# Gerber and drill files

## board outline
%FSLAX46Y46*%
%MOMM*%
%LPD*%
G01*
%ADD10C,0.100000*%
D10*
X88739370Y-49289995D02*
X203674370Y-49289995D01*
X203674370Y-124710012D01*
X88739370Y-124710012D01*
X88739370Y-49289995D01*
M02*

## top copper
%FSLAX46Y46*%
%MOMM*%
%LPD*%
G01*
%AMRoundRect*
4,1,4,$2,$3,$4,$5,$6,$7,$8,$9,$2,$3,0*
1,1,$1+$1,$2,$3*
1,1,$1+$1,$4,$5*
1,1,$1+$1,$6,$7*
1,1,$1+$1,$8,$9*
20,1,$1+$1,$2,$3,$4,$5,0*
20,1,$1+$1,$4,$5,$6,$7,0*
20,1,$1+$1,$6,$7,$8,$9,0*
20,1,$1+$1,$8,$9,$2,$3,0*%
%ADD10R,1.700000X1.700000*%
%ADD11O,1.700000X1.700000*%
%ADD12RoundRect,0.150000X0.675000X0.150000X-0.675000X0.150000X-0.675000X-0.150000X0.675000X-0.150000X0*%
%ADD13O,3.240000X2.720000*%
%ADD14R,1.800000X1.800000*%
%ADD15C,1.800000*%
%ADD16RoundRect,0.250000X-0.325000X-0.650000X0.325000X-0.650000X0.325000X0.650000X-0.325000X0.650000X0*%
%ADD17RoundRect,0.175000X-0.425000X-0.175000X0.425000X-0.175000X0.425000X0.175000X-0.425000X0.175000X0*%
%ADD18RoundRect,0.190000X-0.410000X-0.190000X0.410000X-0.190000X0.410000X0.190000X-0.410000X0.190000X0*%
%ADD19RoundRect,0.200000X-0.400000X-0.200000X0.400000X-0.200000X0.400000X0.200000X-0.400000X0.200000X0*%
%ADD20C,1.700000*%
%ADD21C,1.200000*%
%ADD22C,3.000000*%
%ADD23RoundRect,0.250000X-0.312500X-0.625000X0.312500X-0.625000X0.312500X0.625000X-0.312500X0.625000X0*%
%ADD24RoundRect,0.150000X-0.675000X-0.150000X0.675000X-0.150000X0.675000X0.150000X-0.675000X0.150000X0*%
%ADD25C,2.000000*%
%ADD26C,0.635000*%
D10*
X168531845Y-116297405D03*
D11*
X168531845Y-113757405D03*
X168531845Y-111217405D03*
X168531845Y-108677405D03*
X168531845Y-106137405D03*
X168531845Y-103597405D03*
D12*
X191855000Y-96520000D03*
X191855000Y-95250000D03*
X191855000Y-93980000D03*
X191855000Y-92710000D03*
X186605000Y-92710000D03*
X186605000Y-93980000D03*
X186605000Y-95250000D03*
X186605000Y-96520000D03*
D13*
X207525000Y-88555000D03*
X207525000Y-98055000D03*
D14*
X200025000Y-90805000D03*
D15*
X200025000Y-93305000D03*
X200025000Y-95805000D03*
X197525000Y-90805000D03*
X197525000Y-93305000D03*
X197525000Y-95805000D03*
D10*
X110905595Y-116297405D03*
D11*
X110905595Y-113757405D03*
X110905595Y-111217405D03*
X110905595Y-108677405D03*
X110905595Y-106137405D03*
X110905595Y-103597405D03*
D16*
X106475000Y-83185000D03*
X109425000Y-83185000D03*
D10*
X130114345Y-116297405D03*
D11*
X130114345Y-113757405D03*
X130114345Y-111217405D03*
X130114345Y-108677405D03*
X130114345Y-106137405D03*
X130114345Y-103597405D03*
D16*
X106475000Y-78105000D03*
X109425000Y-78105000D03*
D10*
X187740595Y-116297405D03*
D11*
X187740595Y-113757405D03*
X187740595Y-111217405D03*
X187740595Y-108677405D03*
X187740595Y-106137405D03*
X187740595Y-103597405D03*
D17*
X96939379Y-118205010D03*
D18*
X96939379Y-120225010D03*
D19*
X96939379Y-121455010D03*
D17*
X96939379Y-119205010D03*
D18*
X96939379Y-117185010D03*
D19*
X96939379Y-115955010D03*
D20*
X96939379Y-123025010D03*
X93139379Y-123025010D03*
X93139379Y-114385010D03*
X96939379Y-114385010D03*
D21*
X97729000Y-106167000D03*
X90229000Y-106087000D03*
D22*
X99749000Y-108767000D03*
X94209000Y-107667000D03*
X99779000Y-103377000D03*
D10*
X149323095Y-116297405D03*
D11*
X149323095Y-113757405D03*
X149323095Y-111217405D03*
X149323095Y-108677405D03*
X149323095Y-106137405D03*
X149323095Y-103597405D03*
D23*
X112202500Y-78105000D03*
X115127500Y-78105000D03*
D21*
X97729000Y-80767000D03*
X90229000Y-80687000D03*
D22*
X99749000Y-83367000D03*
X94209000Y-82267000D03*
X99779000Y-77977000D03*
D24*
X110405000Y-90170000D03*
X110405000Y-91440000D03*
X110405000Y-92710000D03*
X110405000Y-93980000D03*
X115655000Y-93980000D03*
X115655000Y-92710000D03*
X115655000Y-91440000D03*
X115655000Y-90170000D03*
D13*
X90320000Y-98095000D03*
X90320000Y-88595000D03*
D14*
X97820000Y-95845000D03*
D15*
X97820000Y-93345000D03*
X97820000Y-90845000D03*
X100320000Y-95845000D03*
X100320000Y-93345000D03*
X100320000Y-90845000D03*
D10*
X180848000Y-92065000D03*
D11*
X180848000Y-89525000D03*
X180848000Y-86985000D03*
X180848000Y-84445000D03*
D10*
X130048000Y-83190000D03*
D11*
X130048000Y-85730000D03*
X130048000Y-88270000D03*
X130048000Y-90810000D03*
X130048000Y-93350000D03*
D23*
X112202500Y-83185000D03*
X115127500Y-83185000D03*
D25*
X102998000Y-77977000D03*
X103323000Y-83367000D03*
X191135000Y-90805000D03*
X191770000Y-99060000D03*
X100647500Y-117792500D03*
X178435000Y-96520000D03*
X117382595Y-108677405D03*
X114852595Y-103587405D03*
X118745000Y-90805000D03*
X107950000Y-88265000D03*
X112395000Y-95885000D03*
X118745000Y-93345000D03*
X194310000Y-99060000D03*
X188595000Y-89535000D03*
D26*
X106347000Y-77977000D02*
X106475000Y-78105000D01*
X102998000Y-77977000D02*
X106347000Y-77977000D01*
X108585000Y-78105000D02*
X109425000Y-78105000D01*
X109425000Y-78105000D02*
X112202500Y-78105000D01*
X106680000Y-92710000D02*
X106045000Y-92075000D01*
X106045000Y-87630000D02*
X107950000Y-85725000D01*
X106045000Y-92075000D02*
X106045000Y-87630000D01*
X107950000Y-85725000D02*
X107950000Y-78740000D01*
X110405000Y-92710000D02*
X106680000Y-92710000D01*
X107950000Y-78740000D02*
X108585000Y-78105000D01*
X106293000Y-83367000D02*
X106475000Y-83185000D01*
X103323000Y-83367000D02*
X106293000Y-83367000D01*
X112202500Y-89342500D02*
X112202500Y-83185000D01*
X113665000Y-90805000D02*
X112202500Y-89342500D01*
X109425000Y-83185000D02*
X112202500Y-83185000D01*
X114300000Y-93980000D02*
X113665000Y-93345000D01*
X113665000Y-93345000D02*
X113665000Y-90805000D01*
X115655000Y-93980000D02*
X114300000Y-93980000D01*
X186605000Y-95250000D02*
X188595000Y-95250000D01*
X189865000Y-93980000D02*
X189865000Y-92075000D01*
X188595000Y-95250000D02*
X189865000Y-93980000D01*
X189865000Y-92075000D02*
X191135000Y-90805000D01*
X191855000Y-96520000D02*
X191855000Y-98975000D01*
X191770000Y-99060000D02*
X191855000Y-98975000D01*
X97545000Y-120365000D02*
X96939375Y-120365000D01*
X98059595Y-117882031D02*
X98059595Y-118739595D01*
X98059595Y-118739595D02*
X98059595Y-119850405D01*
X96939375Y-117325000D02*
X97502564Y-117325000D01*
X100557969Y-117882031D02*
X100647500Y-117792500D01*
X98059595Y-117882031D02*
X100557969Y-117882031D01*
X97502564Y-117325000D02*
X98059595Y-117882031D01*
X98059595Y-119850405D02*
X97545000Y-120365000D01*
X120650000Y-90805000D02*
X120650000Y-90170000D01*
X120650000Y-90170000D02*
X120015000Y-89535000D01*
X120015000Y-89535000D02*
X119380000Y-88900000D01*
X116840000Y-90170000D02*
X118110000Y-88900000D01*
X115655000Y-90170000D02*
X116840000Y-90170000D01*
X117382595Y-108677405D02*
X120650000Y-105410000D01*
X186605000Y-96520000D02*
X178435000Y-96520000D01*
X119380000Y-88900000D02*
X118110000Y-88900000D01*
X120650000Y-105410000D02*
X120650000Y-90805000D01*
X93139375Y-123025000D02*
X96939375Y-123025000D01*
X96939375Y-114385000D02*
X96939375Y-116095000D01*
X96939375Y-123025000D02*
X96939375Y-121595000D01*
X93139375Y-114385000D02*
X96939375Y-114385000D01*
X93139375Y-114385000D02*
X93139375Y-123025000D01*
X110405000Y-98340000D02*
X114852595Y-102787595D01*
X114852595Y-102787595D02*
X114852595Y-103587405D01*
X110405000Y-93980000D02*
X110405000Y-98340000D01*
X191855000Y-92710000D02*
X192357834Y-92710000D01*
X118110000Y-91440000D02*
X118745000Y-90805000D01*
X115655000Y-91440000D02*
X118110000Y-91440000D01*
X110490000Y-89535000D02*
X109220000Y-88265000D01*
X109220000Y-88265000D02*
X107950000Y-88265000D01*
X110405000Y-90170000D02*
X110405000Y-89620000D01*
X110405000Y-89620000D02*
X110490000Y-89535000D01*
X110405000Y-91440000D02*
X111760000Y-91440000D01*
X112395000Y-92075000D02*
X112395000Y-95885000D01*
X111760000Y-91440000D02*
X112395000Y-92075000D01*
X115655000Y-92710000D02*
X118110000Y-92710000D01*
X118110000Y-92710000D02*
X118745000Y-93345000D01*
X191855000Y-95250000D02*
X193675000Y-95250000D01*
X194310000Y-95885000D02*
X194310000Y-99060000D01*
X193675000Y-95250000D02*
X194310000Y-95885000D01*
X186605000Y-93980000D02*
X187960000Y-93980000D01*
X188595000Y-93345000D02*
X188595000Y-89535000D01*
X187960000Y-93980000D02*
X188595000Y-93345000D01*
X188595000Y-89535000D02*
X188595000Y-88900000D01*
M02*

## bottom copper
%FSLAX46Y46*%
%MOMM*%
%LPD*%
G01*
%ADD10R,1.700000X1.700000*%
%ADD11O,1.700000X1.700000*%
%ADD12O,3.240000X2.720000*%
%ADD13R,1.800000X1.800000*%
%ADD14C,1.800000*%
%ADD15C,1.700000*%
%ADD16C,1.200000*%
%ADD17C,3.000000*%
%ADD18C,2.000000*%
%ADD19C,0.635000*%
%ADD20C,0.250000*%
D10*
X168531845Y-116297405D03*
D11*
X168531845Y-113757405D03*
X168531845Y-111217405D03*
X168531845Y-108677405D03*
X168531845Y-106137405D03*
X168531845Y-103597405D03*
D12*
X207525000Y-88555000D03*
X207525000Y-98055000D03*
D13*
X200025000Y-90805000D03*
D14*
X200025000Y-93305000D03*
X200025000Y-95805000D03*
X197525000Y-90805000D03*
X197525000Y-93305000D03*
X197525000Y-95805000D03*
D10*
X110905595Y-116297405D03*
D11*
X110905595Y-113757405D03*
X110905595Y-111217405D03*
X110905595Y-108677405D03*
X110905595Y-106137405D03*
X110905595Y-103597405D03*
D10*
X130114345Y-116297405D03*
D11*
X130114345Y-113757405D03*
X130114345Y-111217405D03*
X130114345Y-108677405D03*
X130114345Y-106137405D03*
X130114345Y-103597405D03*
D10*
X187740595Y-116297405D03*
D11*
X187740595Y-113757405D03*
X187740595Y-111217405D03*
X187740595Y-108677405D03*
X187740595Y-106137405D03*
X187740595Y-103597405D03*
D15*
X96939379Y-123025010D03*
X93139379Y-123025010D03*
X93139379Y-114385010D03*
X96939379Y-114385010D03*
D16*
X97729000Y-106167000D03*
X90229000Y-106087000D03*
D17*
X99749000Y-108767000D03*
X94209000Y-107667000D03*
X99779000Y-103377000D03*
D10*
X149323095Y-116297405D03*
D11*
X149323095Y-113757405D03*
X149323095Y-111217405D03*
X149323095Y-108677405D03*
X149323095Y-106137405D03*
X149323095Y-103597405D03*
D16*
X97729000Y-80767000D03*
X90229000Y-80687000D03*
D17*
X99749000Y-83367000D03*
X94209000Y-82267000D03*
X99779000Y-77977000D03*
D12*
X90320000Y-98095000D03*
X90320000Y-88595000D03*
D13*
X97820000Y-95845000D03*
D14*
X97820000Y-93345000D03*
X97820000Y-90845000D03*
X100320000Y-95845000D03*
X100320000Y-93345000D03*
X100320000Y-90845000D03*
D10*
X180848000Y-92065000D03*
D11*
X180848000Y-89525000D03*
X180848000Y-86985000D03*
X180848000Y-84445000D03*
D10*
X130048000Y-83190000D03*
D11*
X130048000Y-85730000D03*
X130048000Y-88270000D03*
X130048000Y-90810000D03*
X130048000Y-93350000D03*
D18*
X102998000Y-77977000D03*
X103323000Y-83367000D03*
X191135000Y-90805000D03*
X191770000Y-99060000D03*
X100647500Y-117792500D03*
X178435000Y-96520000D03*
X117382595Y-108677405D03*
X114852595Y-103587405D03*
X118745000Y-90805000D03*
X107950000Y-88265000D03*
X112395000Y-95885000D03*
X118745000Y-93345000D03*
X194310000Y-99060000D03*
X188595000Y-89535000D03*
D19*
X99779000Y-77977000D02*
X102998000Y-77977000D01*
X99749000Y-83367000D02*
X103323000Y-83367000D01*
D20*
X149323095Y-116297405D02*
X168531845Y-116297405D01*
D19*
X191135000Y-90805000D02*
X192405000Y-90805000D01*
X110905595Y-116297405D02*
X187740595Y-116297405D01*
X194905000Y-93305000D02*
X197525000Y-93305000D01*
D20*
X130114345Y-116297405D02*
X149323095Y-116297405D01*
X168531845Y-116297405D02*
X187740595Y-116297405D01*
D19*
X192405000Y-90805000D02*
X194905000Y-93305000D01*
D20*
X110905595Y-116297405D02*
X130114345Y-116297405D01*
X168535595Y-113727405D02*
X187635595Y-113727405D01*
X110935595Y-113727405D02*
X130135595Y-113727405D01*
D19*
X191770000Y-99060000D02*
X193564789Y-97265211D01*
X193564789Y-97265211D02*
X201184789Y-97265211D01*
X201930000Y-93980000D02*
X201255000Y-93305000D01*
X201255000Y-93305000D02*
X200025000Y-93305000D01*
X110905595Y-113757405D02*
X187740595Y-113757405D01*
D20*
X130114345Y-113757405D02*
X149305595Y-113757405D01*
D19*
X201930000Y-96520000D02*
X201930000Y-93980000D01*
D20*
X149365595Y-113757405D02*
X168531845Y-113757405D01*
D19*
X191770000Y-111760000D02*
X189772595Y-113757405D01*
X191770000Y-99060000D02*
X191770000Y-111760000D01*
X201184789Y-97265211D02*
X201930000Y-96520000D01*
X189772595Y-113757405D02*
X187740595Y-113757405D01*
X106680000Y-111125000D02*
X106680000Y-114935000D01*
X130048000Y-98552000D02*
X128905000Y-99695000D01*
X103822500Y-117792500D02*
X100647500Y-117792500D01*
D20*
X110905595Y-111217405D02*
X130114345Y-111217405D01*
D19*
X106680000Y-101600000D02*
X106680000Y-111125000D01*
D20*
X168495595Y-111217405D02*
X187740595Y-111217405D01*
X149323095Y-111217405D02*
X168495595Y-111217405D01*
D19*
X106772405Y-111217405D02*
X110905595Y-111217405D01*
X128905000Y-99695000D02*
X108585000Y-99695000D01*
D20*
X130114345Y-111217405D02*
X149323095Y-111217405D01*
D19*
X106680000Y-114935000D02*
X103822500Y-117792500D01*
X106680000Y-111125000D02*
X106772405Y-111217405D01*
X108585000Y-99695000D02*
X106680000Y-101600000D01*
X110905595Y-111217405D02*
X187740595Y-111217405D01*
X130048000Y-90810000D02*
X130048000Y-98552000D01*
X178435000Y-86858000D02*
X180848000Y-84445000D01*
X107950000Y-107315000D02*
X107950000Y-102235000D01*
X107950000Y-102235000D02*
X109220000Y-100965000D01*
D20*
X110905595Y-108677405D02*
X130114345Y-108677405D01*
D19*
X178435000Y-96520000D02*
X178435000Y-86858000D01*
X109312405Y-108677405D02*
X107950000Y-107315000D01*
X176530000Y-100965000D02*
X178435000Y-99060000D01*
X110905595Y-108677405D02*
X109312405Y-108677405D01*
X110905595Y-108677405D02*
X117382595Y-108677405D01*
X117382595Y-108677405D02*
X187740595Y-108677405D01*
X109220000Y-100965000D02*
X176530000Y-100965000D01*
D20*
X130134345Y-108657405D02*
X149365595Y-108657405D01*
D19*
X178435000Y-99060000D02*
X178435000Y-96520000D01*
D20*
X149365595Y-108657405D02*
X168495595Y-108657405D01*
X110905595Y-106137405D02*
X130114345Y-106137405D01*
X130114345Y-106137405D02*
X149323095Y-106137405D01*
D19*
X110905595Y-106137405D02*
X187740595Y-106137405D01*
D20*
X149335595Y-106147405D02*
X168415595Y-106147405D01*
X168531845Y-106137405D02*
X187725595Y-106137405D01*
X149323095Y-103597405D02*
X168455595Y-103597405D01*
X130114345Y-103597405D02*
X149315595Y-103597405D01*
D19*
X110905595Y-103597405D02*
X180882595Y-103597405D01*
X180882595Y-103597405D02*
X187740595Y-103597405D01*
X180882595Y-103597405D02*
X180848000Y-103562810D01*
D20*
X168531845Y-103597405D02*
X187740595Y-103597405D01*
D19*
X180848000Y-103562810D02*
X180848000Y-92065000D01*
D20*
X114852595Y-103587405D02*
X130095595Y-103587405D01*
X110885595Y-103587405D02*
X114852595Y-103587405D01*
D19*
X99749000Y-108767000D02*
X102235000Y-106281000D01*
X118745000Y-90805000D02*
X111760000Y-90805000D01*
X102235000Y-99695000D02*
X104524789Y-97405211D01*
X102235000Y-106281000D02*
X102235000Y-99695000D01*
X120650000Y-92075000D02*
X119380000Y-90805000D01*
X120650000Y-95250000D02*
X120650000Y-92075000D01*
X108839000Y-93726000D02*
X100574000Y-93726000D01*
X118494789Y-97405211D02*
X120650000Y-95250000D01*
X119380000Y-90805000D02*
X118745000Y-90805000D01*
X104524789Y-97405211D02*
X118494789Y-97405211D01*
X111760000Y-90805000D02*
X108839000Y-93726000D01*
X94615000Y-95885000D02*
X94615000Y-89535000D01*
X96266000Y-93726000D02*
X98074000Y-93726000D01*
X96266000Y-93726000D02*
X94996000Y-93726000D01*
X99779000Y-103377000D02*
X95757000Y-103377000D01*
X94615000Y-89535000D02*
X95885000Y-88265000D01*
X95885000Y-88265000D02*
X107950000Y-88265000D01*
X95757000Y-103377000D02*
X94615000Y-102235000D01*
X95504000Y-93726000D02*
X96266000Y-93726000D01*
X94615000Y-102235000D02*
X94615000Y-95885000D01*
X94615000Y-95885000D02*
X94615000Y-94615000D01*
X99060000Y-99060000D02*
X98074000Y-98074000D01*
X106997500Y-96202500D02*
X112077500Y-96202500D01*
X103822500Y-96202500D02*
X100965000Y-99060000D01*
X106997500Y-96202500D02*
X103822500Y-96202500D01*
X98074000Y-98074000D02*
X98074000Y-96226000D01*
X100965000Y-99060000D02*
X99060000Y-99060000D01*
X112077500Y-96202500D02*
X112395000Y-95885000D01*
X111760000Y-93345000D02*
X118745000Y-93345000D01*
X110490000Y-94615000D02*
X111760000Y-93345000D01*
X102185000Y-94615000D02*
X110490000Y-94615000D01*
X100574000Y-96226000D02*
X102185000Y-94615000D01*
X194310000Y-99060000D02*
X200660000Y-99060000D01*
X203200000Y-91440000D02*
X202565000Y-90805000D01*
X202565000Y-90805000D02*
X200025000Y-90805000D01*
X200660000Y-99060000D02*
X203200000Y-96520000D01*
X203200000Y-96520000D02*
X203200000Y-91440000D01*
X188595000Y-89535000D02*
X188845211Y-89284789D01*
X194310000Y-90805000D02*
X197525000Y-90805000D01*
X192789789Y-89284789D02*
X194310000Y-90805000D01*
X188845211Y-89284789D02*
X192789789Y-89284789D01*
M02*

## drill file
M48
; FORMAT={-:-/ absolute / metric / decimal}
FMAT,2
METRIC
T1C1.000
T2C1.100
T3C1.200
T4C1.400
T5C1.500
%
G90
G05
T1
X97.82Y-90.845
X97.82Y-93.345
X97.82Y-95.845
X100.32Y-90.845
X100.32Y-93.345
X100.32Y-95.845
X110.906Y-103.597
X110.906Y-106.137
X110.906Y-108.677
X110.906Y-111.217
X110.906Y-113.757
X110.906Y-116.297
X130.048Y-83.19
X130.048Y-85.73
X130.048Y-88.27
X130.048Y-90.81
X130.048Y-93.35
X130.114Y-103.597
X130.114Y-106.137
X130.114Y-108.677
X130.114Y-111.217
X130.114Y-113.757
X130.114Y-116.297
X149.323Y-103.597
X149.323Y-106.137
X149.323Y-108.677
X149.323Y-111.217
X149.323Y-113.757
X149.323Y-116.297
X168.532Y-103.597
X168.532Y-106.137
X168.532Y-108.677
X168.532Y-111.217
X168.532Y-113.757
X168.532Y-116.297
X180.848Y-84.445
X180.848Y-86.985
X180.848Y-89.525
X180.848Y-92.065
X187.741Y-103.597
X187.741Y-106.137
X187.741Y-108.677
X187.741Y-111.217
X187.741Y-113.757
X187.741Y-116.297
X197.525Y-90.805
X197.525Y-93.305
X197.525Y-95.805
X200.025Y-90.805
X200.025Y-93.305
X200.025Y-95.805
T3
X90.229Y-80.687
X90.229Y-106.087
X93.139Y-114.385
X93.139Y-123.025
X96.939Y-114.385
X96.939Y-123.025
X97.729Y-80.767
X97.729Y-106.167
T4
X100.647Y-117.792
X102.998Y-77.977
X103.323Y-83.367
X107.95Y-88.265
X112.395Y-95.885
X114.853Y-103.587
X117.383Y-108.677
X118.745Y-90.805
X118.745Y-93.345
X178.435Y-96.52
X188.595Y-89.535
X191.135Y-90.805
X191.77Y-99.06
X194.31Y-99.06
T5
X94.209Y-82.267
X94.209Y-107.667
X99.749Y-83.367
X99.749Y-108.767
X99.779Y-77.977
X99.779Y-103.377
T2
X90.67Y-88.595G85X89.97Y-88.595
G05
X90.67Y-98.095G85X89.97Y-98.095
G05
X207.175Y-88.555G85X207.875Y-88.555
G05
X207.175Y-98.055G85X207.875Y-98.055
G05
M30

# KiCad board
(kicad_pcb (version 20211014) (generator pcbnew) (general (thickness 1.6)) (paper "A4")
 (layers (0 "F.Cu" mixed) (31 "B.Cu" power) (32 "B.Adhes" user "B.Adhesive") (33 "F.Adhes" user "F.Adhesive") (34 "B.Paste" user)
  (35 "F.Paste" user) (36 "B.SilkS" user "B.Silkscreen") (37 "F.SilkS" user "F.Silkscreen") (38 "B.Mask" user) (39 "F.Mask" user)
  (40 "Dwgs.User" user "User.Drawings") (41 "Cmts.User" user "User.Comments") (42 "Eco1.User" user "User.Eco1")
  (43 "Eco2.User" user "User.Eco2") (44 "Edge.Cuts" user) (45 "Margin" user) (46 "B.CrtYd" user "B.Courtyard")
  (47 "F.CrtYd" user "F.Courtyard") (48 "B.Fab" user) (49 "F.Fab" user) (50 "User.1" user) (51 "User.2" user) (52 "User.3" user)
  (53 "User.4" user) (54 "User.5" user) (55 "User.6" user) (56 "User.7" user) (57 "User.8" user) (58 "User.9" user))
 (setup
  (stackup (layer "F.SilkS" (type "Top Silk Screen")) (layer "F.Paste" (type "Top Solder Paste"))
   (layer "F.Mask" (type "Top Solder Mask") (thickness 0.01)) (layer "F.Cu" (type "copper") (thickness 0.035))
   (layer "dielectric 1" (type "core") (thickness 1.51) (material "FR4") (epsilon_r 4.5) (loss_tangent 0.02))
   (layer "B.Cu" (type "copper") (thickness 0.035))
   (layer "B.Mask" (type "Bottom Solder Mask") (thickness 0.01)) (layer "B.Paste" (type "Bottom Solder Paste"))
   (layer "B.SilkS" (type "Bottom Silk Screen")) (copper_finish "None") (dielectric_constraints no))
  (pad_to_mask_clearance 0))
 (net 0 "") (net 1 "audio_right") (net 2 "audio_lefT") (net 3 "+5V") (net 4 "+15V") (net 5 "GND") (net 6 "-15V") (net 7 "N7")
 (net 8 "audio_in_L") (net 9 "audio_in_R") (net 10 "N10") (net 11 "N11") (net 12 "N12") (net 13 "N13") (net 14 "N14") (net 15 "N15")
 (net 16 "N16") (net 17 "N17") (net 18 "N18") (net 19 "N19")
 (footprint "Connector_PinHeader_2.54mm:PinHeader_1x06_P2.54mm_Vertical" (layer "F.Cu") (at 168.531845 116.297405 180)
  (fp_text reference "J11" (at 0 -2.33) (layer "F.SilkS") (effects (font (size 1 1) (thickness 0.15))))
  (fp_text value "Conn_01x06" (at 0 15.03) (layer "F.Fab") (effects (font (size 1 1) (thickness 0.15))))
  (pad "1" thru_hole rect (at 0 0 180) (size 1.7 1.7) (drill 1) (layers *.Cu *.Mask) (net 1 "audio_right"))
  (pad "2" thru_hole oval (at 0 2.54 180) (size 1.7 1.7) (drill 1) (layers *.Cu *.Mask) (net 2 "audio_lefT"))
  (pad "3" thru_hole oval (at 0 5.08 180) (size 1.7 1.7) (drill 1) (layers *.Cu *.Mask) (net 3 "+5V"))
  (pad "4" thru_hole oval (at 0 7.62 180) (size 1.7 1.7) (drill 1) (layers *.Cu *.Mask) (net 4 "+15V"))
  (pad "5" thru_hole oval (at 0 10.16 180) (size 1.7 1.7) (drill 1) (layers *.Cu *.Mask) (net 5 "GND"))
  (pad "6" thru_hole oval (at 0 12.7 180) (size 1.7 1.7) (drill 1) (layers *.Cu *.Mask) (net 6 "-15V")))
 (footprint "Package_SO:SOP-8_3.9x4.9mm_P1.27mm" (layer "F.Cu") (at 189.23 94.615 180)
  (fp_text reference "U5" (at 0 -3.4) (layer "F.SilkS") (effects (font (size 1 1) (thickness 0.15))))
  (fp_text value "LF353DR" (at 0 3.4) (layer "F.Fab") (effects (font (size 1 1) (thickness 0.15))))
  (pad "1" smd roundrect (at -2.625 -1.905 180) (size 1.65 0.6) (layers "F.Cu" "F.Paste" "F.Mask") (roundrect_rratio 0.25)
   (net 2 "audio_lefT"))
  (pad "2" smd roundrect (at -2.625 -0.635 180) (size 1.65 0.6) (layers "F.Cu" "F.Paste" "F.Mask") (roundrect_rratio 0.25) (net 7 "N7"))
  (pad "3" smd roundrect (at -2.625 0.635 180) (size 1.65 0.6) (layers "F.Cu" "F.Paste" "F.Mask") (roundrect_rratio 0.25)
   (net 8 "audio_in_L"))
  (pad "4" smd roundrect (at -2.625 1.905 180) (size 1.65 0.6) (layers "F.Cu" "F.Paste" "F.Mask") (roundrect_rratio 0.25) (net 6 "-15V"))
  (pad "5" smd roundrect (at 2.625 1.905 180) (size 1.65 0.6) (layers "F.Cu" "F.Paste" "F.Mask") (roundrect_rratio 0.25)
   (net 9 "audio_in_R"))
  (pad "6" smd roundrect (at 2.625 0.635 180) (size 1.65 0.6) (layers "F.Cu" "F.Paste" "F.Mask") (roundrect_rratio 0.25) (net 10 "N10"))
  (pad "7" smd roundrect (at 2.625 -0.635 180) (size 1.65 0.6) (layers "F.Cu" "F.Paste" "F.Mask") (roundrect_rratio 0.25)
   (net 1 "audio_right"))
  (pad "8" smd roundrect (at 2.625 -1.905 180) (size 1.65 0.6) (layers "F.Cu" "F.Paste" "F.Mask") (roundrect_rratio 0.25) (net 4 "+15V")))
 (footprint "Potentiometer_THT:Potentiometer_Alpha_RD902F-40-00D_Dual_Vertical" (layer "F.Cu") (at 200.025 90.805)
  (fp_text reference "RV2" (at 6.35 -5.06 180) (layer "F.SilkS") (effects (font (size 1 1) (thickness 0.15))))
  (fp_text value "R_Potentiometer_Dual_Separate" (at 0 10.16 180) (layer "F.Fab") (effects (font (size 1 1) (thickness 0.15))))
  (pad "" thru_hole oval (at 7.5 -2.25 90) (size 2.72 3.24) (drill oval 1.1 1.8) (layers *.Cu *.Mask))
  (pad "" thru_hole oval (at 7.5 7.25 90) (size 2.72 3.24) (drill oval 1.1 1.8) (layers *.Cu *.Mask))
  (pad "1" thru_hole rect (at 0 0 90) (size 1.8 1.8) (drill 1) (layers *.Cu *.Mask) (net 7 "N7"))
  (pad "2" thru_hole circle (at 0 2.5 90) (size 1.8 1.8) (drill 1) (layers *.Cu *.Mask) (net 2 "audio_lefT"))
  (pad "3" thru_hole circle (at 0 5 90) (size 1.8 1.8) (drill 1) (layers *.Cu *.Mask) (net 5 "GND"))
  (pad "4" thru_hole circle (at -2.5 0 90) (size 1.8 1.8) (drill 1) (layers *.Cu *.Mask) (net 10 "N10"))
  (pad "5" thru_hole circle (at -2.5 2.5 90) (size 1.8 1.8) (drill 1) (layers *.Cu *.Mask) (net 1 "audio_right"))
  (pad "6" thru_hole circle (at -2.5 5 90) (size 1.8 1.8) (drill 1) (layers *.Cu *.Mask) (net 5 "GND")))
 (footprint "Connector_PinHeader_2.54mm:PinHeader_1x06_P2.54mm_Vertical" (layer "F.Cu") (at 110.905595 116.297405 180)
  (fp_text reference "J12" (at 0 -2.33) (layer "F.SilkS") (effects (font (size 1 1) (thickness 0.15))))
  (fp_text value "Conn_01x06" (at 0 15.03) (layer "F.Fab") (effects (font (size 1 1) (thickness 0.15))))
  (pad "1" thru_hole rect (at 0 0 180) (size 1.7 1.7) (drill 1) (layers *.Cu *.Mask) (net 1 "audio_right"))
  (pad "2" thru_hole oval (at 0 2.54 180) (size 1.7 1.7) (drill 1) (layers *.Cu *.Mask) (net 2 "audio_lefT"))
  (pad "3" thru_hole oval (at 0 5.08 180) (size 1.7 1.7) (drill 1) (layers *.Cu *.Mask) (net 3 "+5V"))
  (pad "4" thru_hole oval (at 0 7.62 180) (size 1.7 1.7) (drill 1) (layers *.Cu *.Mask) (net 4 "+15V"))
  (pad "5" thru_hole oval (at 0 10.16 180) (size 1.7 1.7) (drill 1) (layers *.Cu *.Mask) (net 5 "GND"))
  (pad "6" thru_hole oval (at 0 12.7 180) (size 1.7 1.7) (drill 1) (layers *.Cu *.Mask) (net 6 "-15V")))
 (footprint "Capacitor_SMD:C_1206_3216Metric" (layer "F.Cu") (at 107.95 83.185)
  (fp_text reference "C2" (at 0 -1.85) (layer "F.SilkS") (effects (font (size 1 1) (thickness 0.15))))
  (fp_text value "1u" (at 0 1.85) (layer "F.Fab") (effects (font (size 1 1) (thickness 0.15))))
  (pad "1" smd roundrect (at -1.475 0) (size 1.15 1.8) (layers "F.Cu" "F.Paste" "F.Mask") (roundrect_rratio 0.217391) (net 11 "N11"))
  (pad "2" smd roundrect (at 1.475 0) (size 1.15 1.8) (layers "F.Cu" "F.Paste" "F.Mask") (roundrect_rratio 0.217391) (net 9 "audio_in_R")))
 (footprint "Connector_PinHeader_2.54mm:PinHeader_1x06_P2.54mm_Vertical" (layer "F.Cu") (at 130.114345 116.297405 180)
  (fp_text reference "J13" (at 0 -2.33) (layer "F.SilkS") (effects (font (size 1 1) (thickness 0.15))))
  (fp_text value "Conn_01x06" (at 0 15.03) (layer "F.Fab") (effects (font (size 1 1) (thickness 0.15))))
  (pad "1" thru_hole rect (at 0 0 180) (size 1.7 1.7) (drill 1) (layers *.Cu *.Mask) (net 1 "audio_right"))
  (pad "2" thru_hole oval (at 0 2.54 180) (size 1.7 1.7) (drill 1) (layers *.Cu *.Mask) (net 2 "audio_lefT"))
  (pad "3" thru_hole oval (at 0 5.08 180) (size 1.7 1.7) (drill 1) (layers *.Cu *.Mask) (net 3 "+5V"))
  (pad "4" thru_hole oval (at 0 7.62 180) (size 1.7 1.7) (drill 1) (layers *.Cu *.Mask) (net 4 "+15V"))
  (pad "5" thru_hole oval (at 0 10.16 180) (size 1.7 1.7) (drill 1) (layers *.Cu *.Mask) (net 5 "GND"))
  (pad "6" thru_hole oval (at 0 12.7 180) (size 1.7 1.7) (drill 1) (layers *.Cu *.Mask) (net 6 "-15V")))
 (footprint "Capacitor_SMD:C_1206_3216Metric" (layer "F.Cu") (at 107.95 78.105)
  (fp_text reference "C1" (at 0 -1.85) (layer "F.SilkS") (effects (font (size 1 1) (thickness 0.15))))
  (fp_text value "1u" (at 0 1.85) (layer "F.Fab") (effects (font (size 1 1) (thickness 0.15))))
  (pad "1" smd roundrect (at -1.475 0) (size 1.15 1.8) (layers "F.Cu" "F.Paste" "F.Mask") (roundrect_rratio 0.217391) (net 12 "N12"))
  (pad "2" smd roundrect (at 1.475 0) (size 1.15 1.8) (layers "F.Cu" "F.Paste" "F.Mask") (roundrect_rratio 0.217391) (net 8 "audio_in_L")))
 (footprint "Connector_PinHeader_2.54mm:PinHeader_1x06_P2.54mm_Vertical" (layer "F.Cu") (at 187.740595 116.297405 180)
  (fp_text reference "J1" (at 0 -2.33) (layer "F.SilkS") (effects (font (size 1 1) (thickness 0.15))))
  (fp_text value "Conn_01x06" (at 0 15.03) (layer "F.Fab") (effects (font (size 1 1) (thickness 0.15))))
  (pad "1" thru_hole rect (at 0 0 180) (size 1.7 1.7) (drill 1) (layers *.Cu *.Mask) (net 1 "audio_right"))
  (pad "2" thru_hole oval (at 0 2.54 180) (size 1.7 1.7) (drill 1) (layers *.Cu *.Mask) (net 2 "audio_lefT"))
  (pad "3" thru_hole oval (at 0 5.08 180) (size 1.7 1.7) (drill 1) (layers *.Cu *.Mask) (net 3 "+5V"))
  (pad "4" thru_hole oval (at 0 7.62 180) (size 1.7 1.7) (drill 1) (layers *.Cu *.Mask) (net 4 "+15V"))
  (pad "5" thru_hole oval (at 0 10.16 180) (size 1.7 1.7) (drill 1) (layers *.Cu *.Mask) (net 5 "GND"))
  (pad "6" thru_hole oval (at 0 12.7 180) (size 1.7 1.7) (drill 1) (layers *.Cu *.Mask) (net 6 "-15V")))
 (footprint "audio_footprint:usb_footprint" (layer "F.Cu") (at 96.939379 119.02501 -90)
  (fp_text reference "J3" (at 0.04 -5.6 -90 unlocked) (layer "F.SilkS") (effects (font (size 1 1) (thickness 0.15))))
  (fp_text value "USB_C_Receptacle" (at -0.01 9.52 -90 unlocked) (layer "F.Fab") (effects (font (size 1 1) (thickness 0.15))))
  (pad "A5" smd roundrect (at -0.82 0) (size 1.2 0.7) (layers "F.Cu" "F.Paste" "F.Mask") (roundrect_rratio 0.25) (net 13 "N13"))
  (pad "A9" smd roundrect (at 1.2 0) (size 1.2 0.76) (layers "F.Cu" "F.Paste" "F.Mask") (roundrect_rratio 0.25) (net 3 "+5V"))
  (pad "A12" smd roundrect (at 2.43 0) (size 1.2 0.8) (layers "F.Cu" "F.Paste" "F.Mask") (roundrect_rratio 0.25) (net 5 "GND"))
  (pad "B5" smd roundrect (at 0.18 0) (size 1.2 0.7) (layers "F.Cu" "F.Paste" "F.Mask") (roundrect_rratio 0.25) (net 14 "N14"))
  (pad "B9" smd roundrect (at -1.84 0) (size 1.2 0.76) (layers "F.Cu" "F.Paste" "F.Mask") (roundrect_rratio 0.25) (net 3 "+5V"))
  (pad "B12" smd roundrect (at -3.07 0) (size 1.2 0.8) (layers "F.Cu" "F.Paste" "F.Mask") (roundrect_rratio 0.25) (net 5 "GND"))
  (pad "S1" thru_hole circle (at 4 0) (size 1.7 1.7) (drill 1.2) (layers *.Cu *.Mask) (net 5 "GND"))
  (pad "S1" thru_hole circle (at 4 3.8) (size 1.7 1.7) (drill 1.2) (layers *.Cu *.Mask) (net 5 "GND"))
  (pad "S1" thru_hole circle (at -4.64 3.8) (size 1.7 1.7) (drill 1.2) (layers *.Cu *.Mask) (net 5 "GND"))
  (pad "S1" thru_hole circle (at -4.64 0) (size 1.7 1.7) (drill 1.2) (layers *.Cu *.Mask) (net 5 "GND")))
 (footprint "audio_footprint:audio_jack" (layer "F.Cu") (at 95.25 106.045)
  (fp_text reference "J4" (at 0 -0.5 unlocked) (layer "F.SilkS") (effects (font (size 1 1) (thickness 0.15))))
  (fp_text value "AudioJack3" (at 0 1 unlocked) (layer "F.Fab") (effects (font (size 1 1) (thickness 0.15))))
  (pad "4" thru_hole circle (at 2.479 0.122 90) (size 1.2 1.2) (drill 1.2) (layers *.Cu *.Mask))
  (pad "5" thru_hole circle (at -5.021 0.042 90) (size 1.2 1.2) (drill 1.2) (layers *.Cu *.Mask))
  (pad "R" thru_hole circle (at 4.499 2.722 180) (size 3 3) (drill 1.5) (layers *.Cu *.Mask) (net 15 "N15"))
  (pad "S" thru_hole circle (at -1.041 1.622 90) (size 3 3) (drill 1.5) (layers *.Cu *.Mask) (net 5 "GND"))
  (pad "T" thru_hole circle (at 4.529 -2.668 180) (size 3 3) (drill 1.5) (layers *.Cu *.Mask) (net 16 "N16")))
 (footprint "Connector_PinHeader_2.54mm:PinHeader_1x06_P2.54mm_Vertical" (layer "F.Cu") (at 149.323095 116.297405 180)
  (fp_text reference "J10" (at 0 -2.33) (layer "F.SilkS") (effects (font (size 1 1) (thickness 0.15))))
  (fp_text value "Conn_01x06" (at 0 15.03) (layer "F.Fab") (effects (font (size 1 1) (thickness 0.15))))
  (pad "1" thru_hole rect (at 0 0 180) (size 1.7 1.7) (drill 1) (layers *.Cu *.Mask) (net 1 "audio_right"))
  (pad "2" thru_hole oval (at 0 2.54 180) (size 1.7 1.7) (drill 1) (layers *.Cu *.Mask) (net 2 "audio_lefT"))
  (pad "3" thru_hole oval (at 0 5.08 180) (size 1.7 1.7) (drill 1) (layers *.Cu *.Mask) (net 3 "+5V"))
  (pad "4" thru_hole oval (at 0 7.62 180) (size 1.7 1.7) (drill 1) (layers *.Cu *.Mask) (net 4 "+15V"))
  (pad "5" thru_hole oval (at 0 10.16 180) (size 1.7 1.7) (drill 1) (layers *.Cu *.Mask) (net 5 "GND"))
  (pad "6" thru_hole oval (at 0 12.7 180) (size 1.7 1.7) (drill 1) (layers *.Cu *.Mask) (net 6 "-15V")))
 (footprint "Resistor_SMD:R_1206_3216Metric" (layer "F.Cu") (at 113.665 78.105)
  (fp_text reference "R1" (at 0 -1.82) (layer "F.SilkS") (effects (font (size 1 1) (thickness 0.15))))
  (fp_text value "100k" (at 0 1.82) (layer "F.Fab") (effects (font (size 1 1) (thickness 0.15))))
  (pad "1" smd roundrect (at -1.4625 0) (size 1.125 1.75) (layers "F.Cu" "F.Paste" "F.Mask") (roundrect_rratio 0.222222)
   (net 8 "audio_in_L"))
  (pad "2" smd roundrect (at 1.4625 0) (size 1.125 1.75) (layers "F.Cu" "F.Paste" "F.Mask") (roundrect_rratio 0.222222) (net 5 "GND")))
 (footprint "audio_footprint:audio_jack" (layer "F.Cu") (at 95.25 80.645)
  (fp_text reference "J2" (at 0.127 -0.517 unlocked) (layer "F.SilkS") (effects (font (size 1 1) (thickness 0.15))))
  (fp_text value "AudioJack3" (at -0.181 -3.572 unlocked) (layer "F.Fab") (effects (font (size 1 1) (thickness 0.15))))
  (pad "4" thru_hole circle (at 2.479 0.122 90) (size 1.2 1.2) (drill 1.2) (layers *.Cu *.Mask))
  (pad "5" thru_hole circle (at -5.021 0.042 90) (size 1.2 1.2) (drill 1.2) (layers *.Cu *.Mask))
  (pad "R" thru_hole circle (at 4.499 2.722 180) (size 3 3) (drill 1.5) (layers *.Cu *.Mask) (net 11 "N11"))
  (pad "S" thru_hole circle (at -1.041 1.622 90) (size 3 3) (drill 1.5) (layers *.Cu *.Mask) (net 5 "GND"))
  (pad "T" thru_hole circle (at 4.529 -2.668 180) (size 3 3) (drill 1.5) (layers *.Cu *.Mask) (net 12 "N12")))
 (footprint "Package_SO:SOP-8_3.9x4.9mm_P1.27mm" (layer "F.Cu") (at 113.03 92.075)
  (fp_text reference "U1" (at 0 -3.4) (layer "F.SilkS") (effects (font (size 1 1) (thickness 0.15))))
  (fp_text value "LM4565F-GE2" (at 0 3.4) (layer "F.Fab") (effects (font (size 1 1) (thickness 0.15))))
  (pad "1" smd roundrect (at -2.625 -1.905) (size 1.65 0.6) (layers "F.Cu" "F.Paste" "F.Mask") (roundrect_rratio 0.25) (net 16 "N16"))
  (pad "2" smd roundrect (at -2.625 -0.635) (size 1.65 0.6) (layers "F.Cu" "F.Paste" "F.Mask") (roundrect_rratio 0.25) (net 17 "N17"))
  (pad "3" smd roundrect (at -2.625 0.635) (size 1.65 0.6) (layers "F.Cu" "F.Paste" "F.Mask") (roundrect_rratio 0.25) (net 8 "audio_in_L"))
  (pad "4" smd roundrect (at -2.625 1.905) (size 1.65 0.6) (layers "F.Cu" "F.Paste" "F.Mask") (roundrect_rratio 0.25) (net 6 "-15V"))
  (pad "5" smd roundrect (at 2.625 1.905) (size 1.65 0.6) (layers "F.Cu" "F.Paste" "F.Mask") (roundrect_rratio 0.25) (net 9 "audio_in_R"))
  (pad "6" smd roundrect (at 2.625 0.635) (size 1.65 0.6) (layers "F.Cu" "F.Paste" "F.Mask") (roundrect_rratio 0.25) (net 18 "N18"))
  (pad "7" smd roundrect (at 2.625 -0.635) (size 1.65 0.6) (layers "F.Cu" "F.Paste" "F.Mask") (roundrect_rratio 0.25) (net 15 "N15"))
  (pad "8" smd roundrect (at 2.625 -1.905) (size 1.65 0.6) (layers "F.Cu" "F.Paste" "F.Mask") (roundrect_rratio 0.25) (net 4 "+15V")))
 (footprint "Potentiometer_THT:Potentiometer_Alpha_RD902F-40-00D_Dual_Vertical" (layer "F.Cu") (at 97.82 95.845 180)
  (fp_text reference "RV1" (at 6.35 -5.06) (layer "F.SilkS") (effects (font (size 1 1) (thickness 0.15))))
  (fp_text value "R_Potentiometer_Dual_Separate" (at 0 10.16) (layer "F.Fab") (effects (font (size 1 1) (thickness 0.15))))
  (pad "" thru_hole oval (at 7.5 -2.25 270) (size 2.72 3.24) (drill oval 1.1 1.8) (layers *.Cu *.Mask))
  (pad "" thru_hole oval (at 7.5 7.25 270) (size 2.72 3.24) (drill oval 1.1 1.8) (layers *.Cu *.Mask))
  (pad "1" thru_hole rect (at 0 0 270) (size 1.8 1.8) (drill 1) (layers *.Cu *.Mask) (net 17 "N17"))
  (pad "2" thru_hole circle (at 0 2.5 270) (size 1.8 1.8) (drill 1) (layers *.Cu *.Mask) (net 16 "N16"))
  (pad "3" thru_hole circle (at 0 5 270) (size 1.8 1.8) (drill 1) (layers *.Cu *.Mask) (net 5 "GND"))
  (pad "4" thru_hole circle (at -2.5 0 270) (size 1.8 1.8) (drill 1) (layers *.Cu *.Mask) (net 18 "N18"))
  (pad "5" thru_hole circle (at -2.5 2.5 270) (size 1.8 1.8) (drill 1) (layers *.Cu *.Mask) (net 15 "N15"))
  (pad "6" thru_hole circle (at -2.5 5 270) (size 1.8 1.8) (drill 1) (layers *.Cu *.Mask) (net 5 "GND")))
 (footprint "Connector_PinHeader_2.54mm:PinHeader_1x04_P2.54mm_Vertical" (layer "F.Cu") (at 180.848 92.065 180)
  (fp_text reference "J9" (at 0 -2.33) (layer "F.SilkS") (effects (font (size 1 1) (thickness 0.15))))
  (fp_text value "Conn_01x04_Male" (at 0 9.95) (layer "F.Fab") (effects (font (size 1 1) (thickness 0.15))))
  (pad "1" thru_hole rect (at 0 0 180) (size 1.7 1.7) (drill 1) (layers *.Cu *.Mask) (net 6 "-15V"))
  (pad "2" thru_hole oval (at 0 2.54 180) (size 1.7 1.7) (drill 1) (layers *.Cu *.Mask) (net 5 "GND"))
  (pad "3" thru_hole oval (at 0 5.08 180) (size 1.7 1.7) (drill 1) (layers *.Cu *.Mask) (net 5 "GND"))
  (pad "4" thru_hole oval (at 0 7.62 180) (size 1.7 1.7) (drill 1) (layers *.Cu *.Mask) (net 4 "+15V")))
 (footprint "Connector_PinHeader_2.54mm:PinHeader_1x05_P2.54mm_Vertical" (layer "F.Cu") (at 130.048 83.19)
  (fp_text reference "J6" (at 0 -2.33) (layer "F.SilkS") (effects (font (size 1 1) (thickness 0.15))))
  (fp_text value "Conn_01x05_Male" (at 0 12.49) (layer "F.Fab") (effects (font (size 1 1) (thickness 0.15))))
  (pad "1" thru_hole rect (at 0 0) (size 1.7 1.7) (drill 1) (layers *.Cu *.Mask) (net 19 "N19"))
  (pad "2" thru_hole oval (at 0 2.54) (size 1.7 1.7) (drill 1) (layers *.Cu *.Mask) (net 5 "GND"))
  (pad "3" thru_hole oval (at 0 5.08) (size 1.7 1.7) (drill 1) (layers *.Cu *.Mask) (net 5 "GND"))
  (pad "4" thru_hole oval (at 0 7.62) (size 1.7 1.7) (drill 1) (layers *.Cu *.Mask) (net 3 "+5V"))
  (pad "5" thru_hole oval (at 0 10.16) (size 1.7 1.7) (drill 1) (layers *.Cu *.Mask) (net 3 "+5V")))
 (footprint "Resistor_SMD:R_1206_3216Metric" (layer "F.Cu") (at 113.665 83.185)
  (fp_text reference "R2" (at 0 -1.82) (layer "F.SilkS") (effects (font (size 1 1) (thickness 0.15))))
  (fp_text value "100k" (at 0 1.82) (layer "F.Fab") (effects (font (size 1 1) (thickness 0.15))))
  (pad "1" smd roundrect (at -1.4625 0) (size 1.125 1.75) (layers "F.Cu" "F.Paste" "F.Mask") (roundrect_rratio 0.222222)
   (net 9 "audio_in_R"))
  (pad "2" smd roundrect (at 1.4625 0) (size 1.125 1.75) (layers "F.Cu" "F.Paste" "F.Mask") (roundrect_rratio 0.222222) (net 5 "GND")))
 (gr_rect locked (start 88.73937 49.289995) (end 203.67437 124.710012) (layer "Edge.Cuts") (width 0.1) (fill none))
 (segment (start 106.347 77.977) (end 106.475 78.105) (width 0.635) (layer "F.Cu") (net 12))
 (segment (start 102.998 77.977) (end 106.347 77.977) (width 0.635) (layer "F.Cu") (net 12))
 (via (at 102.998 77.977) (size 2) (drill 1.4) (layers "F.Cu" "B.Cu") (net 12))
 (segment (start 99.779 77.977) (end 102.998 77.977) (width 0.635) (layer "B.Cu") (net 12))
 (segment (start 108.585 78.105) (end 109.425 78.105) (width 0.635) (layer "F.Cu") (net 8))
 (segment (start 109.425 78.105) (end 112.2025 78.105) (width 0.635) (layer "F.Cu") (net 8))
 (segment (start 106.68 92.71) (end 106.045 92.075) (width 0.635) (layer "F.Cu") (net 8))
 (segment (start 106.045 87.63) (end 107.95 85.725) (width 0.635) (layer "F.Cu") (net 8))
 (segment (start 106.045 92.075) (end 106.045 87.63) (width 0.635) (layer "F.Cu") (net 8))
 (segment (start 107.95 85.725) (end 107.95 78.74) (width 0.635) (layer "F.Cu") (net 8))
 (segment (start 110.405 92.71) (end 106.68 92.71) (width 0.635) (layer "F.Cu") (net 8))
 (segment (start 107.95 78.74) (end 108.585 78.105) (width 0.635) (layer "F.Cu") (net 8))
 (segment (start 106.293 83.367) (end 106.475 83.185) (width 0.635) (layer "F.Cu") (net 11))
 (segment (start 103.323 83.367) (end 106.293 83.367) (width 0.635) (layer "F.Cu") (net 11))
 (via (at 103.323 83.367) (size 2) (drill 1.4) (layers "F.Cu" "B.Cu") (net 11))
 (segment (start 99.749 83.367) (end 103.323 83.367) (width 0.635) (layer "B.Cu") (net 11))
 (segment (start 112.2025 89.3425) (end 112.2025 83.185) (width 0.635) (layer "F.Cu") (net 9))
 (segment (start 113.665 90.805) (end 112.2025 89.3425) (width 0.635) (layer "F.Cu") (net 9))
 (segment (start 109.425 83.185) (end 112.2025 83.185) (width 0.635) (layer "F.Cu") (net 9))
 (segment (start 114.3 93.98) (end 113.665 93.345) (width 0.635) (layer "F.Cu") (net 9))
 (segment (start 113.665 93.345) (end 113.665 90.805) (width 0.635) (layer "F.Cu") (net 9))
 (segment (start 115.655 93.98) (end 114.3 93.98) (width 0.635) (layer "F.Cu") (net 9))
 (segment (start 186.605 95.25) (end 188.595 95.25) (width 0.635) (layer "F.Cu") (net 1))
 (segment (start 189.865 93.98) (end 189.865 92.075) (width 0.635) (layer "F.Cu") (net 1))
 (segment (start 188.595 95.25) (end 189.865 93.98) (width 0.635) (layer "F.Cu") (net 1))
 (segment (start 189.865 92.075) (end 191.135 90.805) (width 0.635) (layer "F.Cu") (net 1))
 (via (at 191.135 90.805) (size 2) (drill 1.4) (layers "F.Cu" "B.Cu") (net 1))
 (segment (start 149.323095 116.297405) (end 168.531845 116.297405) (width 0.25) (layer "B.Cu") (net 1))
 (segment (start 191.135 90.805) (end 192.405 90.805) (width 0.635) (layer "B.Cu") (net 1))
 (segment (start 110.905595 116.297405) (end 187.740595 116.297405) (width 0.635) (layer "B.Cu") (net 1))
 (segment (start 194.905 93.305) (end 197.525 93.305) (width 0.635) (layer "B.Cu") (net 1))
 (segment (start 130.114345 116.297405) (end 149.323095 116.297405) (width 0.25) (layer "B.Cu") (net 1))
 (segment (start 168.531845 116.297405) (end 187.740595 116.297405) (width 0.25) (layer "B.Cu") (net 1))
 (segment (start 192.405 90.805) (end 194.905 93.305) (width 0.635) (layer "B.Cu") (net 1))
 (segment (start 110.905595 116.297405) (end 130.114345 116.297405) (width 0.25) (layer "B.Cu") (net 1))
 (segment (start 191.855 96.52) (end 191.855 98.975) (width 0.635) (layer "F.Cu") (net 2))
 (segment (start 191.77 99.06) (end 191.855 98.975) (width 0.635) (layer "F.Cu") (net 2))
 (via (at 191.77 99.06) (size 2) (drill 1.4) (layers "F.Cu" "B.Cu") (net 2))
 (segment (start 168.535595 113.727405) (end 187.635595 113.727405) (width 0.25) (layer "B.Cu") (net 2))
 (segment (start 110.935595 113.727405) (end 130.135595 113.727405) (width 0.25) (layer "B.Cu") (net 2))
 (segment (start 191.77 99.06) (end 193.564789 97.265211) (width 0.635) (layer "B.Cu") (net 2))
 (segment (start 193.564789 97.265211) (end 201.184789 97.265211) (width 0.635) (layer "B.Cu") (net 2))
 (segment (start 201.93 93.98) (end 201.255 93.305) (width 0.635) (layer "B.Cu") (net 2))
 (segment (start 201.255 93.305) (end 200.025 93.305) (width 0.635) (layer "B.Cu") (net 2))
 (segment (start 110.905595 113.757405) (end 187.740595 113.757405) (width 0.635) (layer "B.Cu") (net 2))
 (segment (start 130.114345 113.757405) (end 149.305595 113.757405) (width 0.25) (layer "B.Cu") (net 2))
 (segment (start 201.93 96.52) (end 201.93 93.98) (width 0.635) (layer "B.Cu") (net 2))
 (segment (start 149.365595 113.757405) (end 168.531845 113.757405) (width 0.25) (layer "B.Cu") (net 2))
 (segment (start 191.77 111.76) (end 189.772595 113.757405) (width 0.635) (layer "B.Cu") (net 2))
 (segment (start 191.77 99.06) (end 191.77 111.76) (width 0.635) (layer "B.Cu") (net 2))
 (segment (start 201.184789 97.265211) (end 201.93 96.52) (width 0.635) (layer "B.Cu") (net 2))
 (segment (start 189.772595 113.757405) (end 187.740595 113.757405) (width 0.635) (layer "B.Cu") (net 2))
 (segment (start 97.545 120.365) (end 96.939375 120.365) (width 0.635) (layer "F.Cu") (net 3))
 (segment (start 98.059595 117.882031) (end 98.059595 118.739595) (width 0.635) (layer "F.Cu") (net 3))
 (segment (start 98.059595 118.739595) (end 98.059595 119.850405) (width 0.635) (layer "F.Cu") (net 3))
 (segment (start 96.939375 117.325) (end 97.502564 117.325) (width 0.635) (layer "F.Cu") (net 3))
 (segment (start 100.557969 117.882031) (end 100.6475 117.7925) (width 0.635) (layer "F.Cu") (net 3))
 (segment (start 98.059595 117.882031) (end 100.557969 117.882031) (width 0.635) (layer "F.Cu") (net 3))
 (segment (start 97.502564 117.325) (end 98.059595 117.882031) (width 0.635) (layer "F.Cu") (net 3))
 (segment (start 98.059595 119.850405) (end 97.545 120.365) (width 0.635) (layer "F.Cu") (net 3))
 (via (at 100.6475 117.7925) (size 2) (drill 1.4) (layers "F.Cu" "B.Cu") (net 3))
 (segment (start 106.68 111.125) (end 106.68 114.935) (width 0.635) (layer "B.Cu") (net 3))
 (segment (start 130.048 98.552) (end 128.905 99.695) (width 0.635) (layer "B.Cu") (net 3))
 (segment (start 103.8225 117.7925) (end 100.6475 117.7925) (width 0.635) (layer "B.Cu") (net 3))
 (segment (start 110.905595 111.217405) (end 130.114345 111.217405) (width 0.25) (layer "B.Cu") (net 3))
 (segment (start 106.68 101.6) (end 106.68 111.125) (width 0.635) (layer "B.Cu") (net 3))
 (segment (start 168.495595 111.217405) (end 187.740595 111.217405) (width 0.25) (layer "B.Cu") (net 3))
 (segment (start 149.323095 111.217405) (end 168.495595 111.217405) (width 0.25) (layer "B.Cu") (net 3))
 (segment (start 106.772405 111.217405) (end 110.905595 111.217405) (width 0.635) (layer "B.Cu") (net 3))
 (segment (start 128.905 99.695) (end 108.585 99.695) (width 0.635) (layer "B.Cu") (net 3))
 (segment (start 130.114345 111.217405) (end 149.323095 111.217405) (width 0.25) (layer "B.Cu") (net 3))
 (segment (start 106.68 114.935) (end 103.8225 117.7925) (width 0.635) (layer "B.Cu") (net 3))
 (segment (start 106.68 111.125) (end 106.772405 111.217405) (width 0.635) (layer "B.Cu") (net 3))
 (segment (start 108.585 99.695) (end 106.68 101.6) (width 0.635) (layer "B.Cu") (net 3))
 (segment (start 110.905595 111.217405) (end 187.740595 111.217405) (width 0.635) (layer "B.Cu") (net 3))
 (segment (start 130.048 90.81) (end 130.048 98.552) (width 0.635) (layer "B.Cu") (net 3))
 (segment (start 120.65 90.805) (end 120.65 90.17) (width 0.635) (layer "F.Cu") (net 4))
 (segment (start 120.65 90.17) (end 120.015 89.535) (width 0.635) (layer "F.Cu") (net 4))
 (segment (start 120.015 89.535) (end 119.38 88.9) (width 0.635) (layer "F.Cu") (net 4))
 (segment (start 116.84 90.17) (end 118.11 88.9) (width 0.635) (layer "F.Cu") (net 4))
 (segment (start 115.655 90.17) (end 116.84 90.17) (width 0.635) (layer "F.Cu") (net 4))
 (segment (start 117.382595 108.677405) (end 120.65 105.41) (width 0.635) (layer "F.Cu") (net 4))
 (segment (start 186.605 96.52) (end 178.435 96.52) (width 0.635) (layer "F.Cu") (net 4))
 (segment (start 119.38 88.9) (end 118.11 88.9) (width 0.635) (layer "F.Cu") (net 4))
 (segment (start 120.65 105.41) (end 120.65 90.805) (width 0.635) (layer "F.Cu") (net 4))
 (via (at 178.435 96.52) (size 2) (drill 1.4) (layers "F.Cu" "B.Cu") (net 4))
 (via (at 117.382595 108.677405) (size 2) (drill 1.4) (layers "F.Cu" "B.Cu") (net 4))
 (segment (start 178.435 86.858) (end 180.848 84.445) (width 0.635) (layer "B.Cu") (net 4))
 (segment (start 107.95 107.315) (end 107.95 102.235) (width 0.635) (layer "B.Cu") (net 4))
 (segment (start 107.95 102.235) (end 109.22 100.965) (width 0.635) (layer "B.Cu") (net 4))
 (segment (start 110.905595 108.677405) (end 130.114345 108.677405) (width 0.25) (layer "B.Cu") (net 4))
 (segment (start 178.435 96.52) (end 178.435 86.858) (width 0.635) (layer "B.Cu") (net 4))
 (segment (start 109.312405 108.677405) (end 107.95 107.315) (width 0.635) (layer "B.Cu") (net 4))
 (segment (start 176.53 100.965) (end 178.435 99.06) (width 0.635) (layer "B.Cu") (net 4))
 (segment (start 110.905595 108.677405) (end 109.312405 108.677405) (width 0.635) (layer "B.Cu") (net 4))
 (segment (start 110.905595 108.677405) (end 117.382595 108.677405) (width 0.635) (layer "B.Cu") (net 4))
 (segment (start 117.382595 108.677405) (end 187.740595 108.677405) (width 0.635) (layer "B.Cu") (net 4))
 (segment (start 109.22 100.965) (end 176.53 100.965) (width 0.635) (layer "B.Cu") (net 4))
 (segment (start 130.134345 108.657405) (end 149.365595 108.657405) (width 0.25) (layer "B.Cu") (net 4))
 (segment (start 178.435 99.06) (end 178.435 96.52) (width 0.635) (layer "B.Cu") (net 4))
 (segment (start 149.365595 108.657405) (end 168.495595 108.657405) (width 0.25) (layer "B.Cu") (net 4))
 (segment (start 93.139375 123.025) (end 96.939375 123.025) (width 0.635) (layer "F.Cu") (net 5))
 (segment (start 96.939375 114.385) (end 96.939375 116.095) (width 0.635) (layer "F.Cu") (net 5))
 (segment (start 96.939375 123.025) (end 96.939375 121.595) (width 0.635) (layer "F.Cu") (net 5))
 (segment (start 93.139375 114.385) (end 96.939375 114.385) (width 0.635) (layer "F.Cu") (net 5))
 (segment (start 93.139375 114.385) (end 93.139375 123.025) (width 0.635) (layer "F.Cu") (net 5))
 (segment (start 110.905595 106.137405) (end 130.114345 106.137405) (width 0.25) (layer "B.Cu") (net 5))
 (segment (start 130.114345 106.137405) (end 149.323095 106.137405) (width 0.25) (layer "B.Cu") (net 5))
 (segment (start 110.905595 106.137405) (end 187.740595 106.137405) (width 0.635) (layer "B.Cu") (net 5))
 (segment (start 149.335595 106.147405) (end 168.415595 106.147405) (width 0.25) (layer "B.Cu") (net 5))
 (segment (start 168.531845 106.137405) (end 187.725595 106.137405) (width 0.25) (layer "B.Cu") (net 5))
 (segment (start 110.405 98.34) (end 114.852595 102.787595) (width 0.635) (layer "F.Cu") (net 6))
 (segment (start 114.852595 102.787595) (end 114.852595 103.587405) (width 0.635) (layer "F.Cu") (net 6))
 (segment (start 110.405 93.98) (end 110.405 98.34) (width 0.635) (layer "F.Cu") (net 6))
 (segment (start 191.855 92.71) (end 192.357834 92.71) (width 0.635) (layer "F.Cu") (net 6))
 (via (at 114.852595 103.587405) (size 2) (drill 1.4) (layers "F.Cu" "B.Cu") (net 6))
 (segment (start 149.323095 103.597405) (end 168.455595 103.597405) (width 0.25) (layer "B.Cu") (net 6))
 (segment (start 130.114345 103.597405) (end 149.315595 103.597405) (width 0.25) (layer "B.Cu") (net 6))
 (segment (start 110.905595 103.597405) (end 180.882595 103.597405) (width 0.635) (layer "B.Cu") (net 6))
 (segment (start 180.882595 103.597405) (end 187.740595 103.597405) (width 0.635) (layer "B.Cu") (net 6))
 (segment (start 180.882595 103.597405) (end 180.848 103.56281) (width 0.635) (layer "B.Cu") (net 6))
 (segment (start 168.531845 103.597405) (end 187.740595 103.597405) (width 0.25) (layer "B.Cu") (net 6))
 (segment (start 180.848 103.56281) (end 180.848 92.065) (width 0.635) (layer "B.Cu") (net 6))
 (segment (start 114.852595 103.587405) (end 130.095595 103.587405) (width 0.25) (layer "B.Cu") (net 6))
 (segment (start 110.885595 103.587405) (end 114.852595 103.587405) (width 0.25) (layer "B.Cu") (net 6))
 (segment (start 118.11 91.44) (end 118.745 90.805) (width 0.635) (layer "F.Cu") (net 15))
 (segment (start 115.655 91.44) (end 118.11 91.44) (width 0.635) (layer "F.Cu") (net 15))
 (via (at 118.745 90.805) (size 2) (drill 1.4) (layers "F.Cu" "B.Cu") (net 15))
 (segment (start 99.749 108.767) (end 102.235 106.281) (width 0.635) (layer "B.Cu") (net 15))
 (segment (start 118.745 90.805) (end 111.76 90.805) (width 0.635) (layer "B.Cu") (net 15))
 (segment (start 102.235 99.695) (end 104.524789 97.405211) (width 0.635) (layer "B.Cu") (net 15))
 (segment (start 102.235 106.281) (end 102.235 99.695) (width 0.635) (layer "B.Cu") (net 15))
 (segment (start 120.65 92.075) (end 119.38 90.805) (width 0.635) (layer "B.Cu") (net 15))
 (segment (start 120.65 95.25) (end 120.65 92.075) (width 0.635) (layer "B.Cu") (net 15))
 (segment (start 108.839 93.726) (end 100.574 93.726) (width 0.635) (layer "B.Cu") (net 15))
 (segment (start 118.494789 97.405211) (end 120.65 95.25) (width 0.635) (layer "B.Cu") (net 15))
 (segment (start 119.38 90.805) (end 118.745 90.805) (width 0.635) (layer "B.Cu") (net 15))
 (segment (start 104.524789 97.405211) (end 118.494789 97.405211) (width 0.635) (layer "B.Cu") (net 15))
 (segment (start 111.76 90.805) (end 108.839 93.726) (width 0.635) (layer "B.Cu") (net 15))
 (segment (start 110.49 89.535) (end 109.22 88.265) (width 0.635) (layer "F.Cu") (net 16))
 (segment (start 109.22 88.265) (end 107.95 88.265) (width 0.635) (layer "F.Cu") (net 16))
 (segment (start 110.405 90.17) (end 110.405 89.62) (width 0.635) (layer "F.Cu") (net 16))
 (segment (start 110.405 89.62) (end 110.49 89.535) (width 0.635) (layer "F.Cu") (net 16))
 (via (at 107.95 88.265) (size 2) (drill 1.4) (layers "F.Cu" "B.Cu") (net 16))
 (segment (start 94.615 95.885) (end 94.615 89.535) (width 0.635) (layer "B.Cu") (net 16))
 (segment (start 96.266 93.726) (end 98.074 93.726) (width 0.635) (layer "B.Cu") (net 16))
 (segment (start 96.266 93.726) (end 94.996 93.726) (width 0.635) (layer "B.Cu") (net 16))
 (segment (start 99.779 103.377) (end 95.757 103.377) (width 0.635) (layer "B.Cu") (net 16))
 (segment (start 94.615 89.535) (end 95.885 88.265) (width 0.635) (layer "B.Cu") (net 16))
 (segment (start 95.885 88.265) (end 107.95 88.265) (width 0.635) (layer "B.Cu") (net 16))
 (segment (start 95.757 103.377) (end 94.615 102.235) (width 0.635) (layer "B.Cu") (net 16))
 (segment (start 95.504 93.726) (end 96.266 93.726) (width 0.635) (layer "B.Cu") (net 16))
 (segment (start 94.615 102.235) (end 94.615 95.885) (width 0.635) (layer "B.Cu") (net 16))
 (segment (start 94.615 95.885) (end 94.615 94.615) (width 0.635) (layer "B.Cu") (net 16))
 (segment (start 110.405 91.44) (end 111.76 91.44) (width 0.635) (layer "F.Cu") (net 17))
 (segment (start 112.395 92.075) (end 112.395 95.885) (width 0.635) (layer "F.Cu") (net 17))
 (segment (start 111.76 91.44) (end 112.395 92.075) (width 0.635) (layer "F.Cu") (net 17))
 (via (at 112.395 95.885) (size 2) (drill 1.4) (layers "F.Cu" "B.Cu") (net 17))
 (segment (start 99.06 99.06) (end 98.074 98.074) (width 0.635) (layer "B.Cu") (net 17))
 (segment (start 106.9975 96.2025) (end 112.0775 96.2025) (width 0.635) (layer "B.Cu") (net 17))
 (segment (start 103.8225 96.2025) (end 100.965 99.06) (width 0.635) (layer "B.Cu") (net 17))
 (segment (start 106.9975 96.2025) (end 103.8225 96.2025) (width 0.635) (layer "B.Cu") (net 17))
 (segment (start 98.074 98.074) (end 98.074 96.226) (width 0.635) (layer "B.Cu") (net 17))
 (segment (start 100.965 99.06) (end 99.06 99.06) (width 0.635) (layer "B.Cu") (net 17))
 (segment (start 112.0775 96.2025) (end 112.395 95.885) (width 0.635) (layer "B.Cu") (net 17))
 (segment (start 115.655 92.71) (end 118.11 92.71) (width 0.635) (layer "F.Cu") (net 18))
 (segment (start 118.11 92.71) (end 118.745 93.345) (width 0.635) (layer "F.Cu") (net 18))
 (via (at 118.745 93.345) (size 2) (drill 1.4) (layers "F.Cu" "B.Cu") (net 18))
 (segment (start 111.76 93.345) (end 118.745 93.345) (width 0.635) (layer "B.Cu") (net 18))
 (segment (start 110.49 94.615) (end 111.76 93.345) (width 0.635) (layer "B.Cu") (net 18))
 (segment (start 102.185 94.615) (end 110.49 94.615) (width 0.635) (layer "B.Cu") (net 18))
 (segment (start 100.574 96.226) (end 102.185 94.615) (width 0.635) (layer "B.Cu") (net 18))
 (segment (start 191.855 95.25) (end 193.675 95.25) (width 0.635) (layer "F.Cu") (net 7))
 (segment (start 194.31 95.885) (end 194.31 99.06) (width 0.635) (layer "F.Cu") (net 7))
 (segment (start 193.675 95.25) (end 194.31 95.885) (width 0.635) (layer "F.Cu") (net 7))
 (via (at 194.31 99.06) (size 2) (drill 1.4) (layers "F.Cu" "B.Cu") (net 7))
 (segment (start 194.31 99.06) (end 200.66 99.06) (width 0.635) (layer "B.Cu") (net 7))
 (segment (start 203.2 91.44) (end 202.565 90.805) (width 0.635) (layer "B.Cu") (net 7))
 (segment (start 202.565 90.805) (end 200.025 90.805) (width 0.635) (layer "B.Cu") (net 7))
 (segment (start 200.66 99.06) (end 203.2 96.52) (width 0.635) (layer "B.Cu") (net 7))
 (segment (start 203.2 96.52) (end 203.2 91.44) (width 0.635) (layer "B.Cu") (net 7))
 (segment (start 186.605 93.98) (end 187.96 93.98) (width 0.635) (layer "F.Cu") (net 10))
 (segment (start 188.595 93.345) (end 188.595 89.535) (width 0.635) (layer "F.Cu") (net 10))
 (segment (start 187.96 93.98) (end 188.595 93.345) (width 0.635) (layer "F.Cu") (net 10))
 (segment (start 188.595 89.535) (end 188.595 88.9) (width 0.635) (layer "F.Cu") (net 10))
 (via (at 188.595 89.535) (size 2) (drill 1.4) (layers "F.Cu" "B.Cu") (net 10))
 (segment (start 188.595 89.535) (end 188.845211 89.284789) (width 0.635) (layer "B.Cu") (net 10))
 (segment (start 194.31 90.805) (end 197.525 90.805) (width 0.635) (layer "B.Cu") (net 10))
 (segment (start 192.789789 89.284789) (end 194.31 90.805) (width 0.635) (layer "B.Cu") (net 10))
 (segment (start 188.845211 89.284789) (end 192.789789 89.284789) (width 0.635) (layer "B.Cu") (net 10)))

